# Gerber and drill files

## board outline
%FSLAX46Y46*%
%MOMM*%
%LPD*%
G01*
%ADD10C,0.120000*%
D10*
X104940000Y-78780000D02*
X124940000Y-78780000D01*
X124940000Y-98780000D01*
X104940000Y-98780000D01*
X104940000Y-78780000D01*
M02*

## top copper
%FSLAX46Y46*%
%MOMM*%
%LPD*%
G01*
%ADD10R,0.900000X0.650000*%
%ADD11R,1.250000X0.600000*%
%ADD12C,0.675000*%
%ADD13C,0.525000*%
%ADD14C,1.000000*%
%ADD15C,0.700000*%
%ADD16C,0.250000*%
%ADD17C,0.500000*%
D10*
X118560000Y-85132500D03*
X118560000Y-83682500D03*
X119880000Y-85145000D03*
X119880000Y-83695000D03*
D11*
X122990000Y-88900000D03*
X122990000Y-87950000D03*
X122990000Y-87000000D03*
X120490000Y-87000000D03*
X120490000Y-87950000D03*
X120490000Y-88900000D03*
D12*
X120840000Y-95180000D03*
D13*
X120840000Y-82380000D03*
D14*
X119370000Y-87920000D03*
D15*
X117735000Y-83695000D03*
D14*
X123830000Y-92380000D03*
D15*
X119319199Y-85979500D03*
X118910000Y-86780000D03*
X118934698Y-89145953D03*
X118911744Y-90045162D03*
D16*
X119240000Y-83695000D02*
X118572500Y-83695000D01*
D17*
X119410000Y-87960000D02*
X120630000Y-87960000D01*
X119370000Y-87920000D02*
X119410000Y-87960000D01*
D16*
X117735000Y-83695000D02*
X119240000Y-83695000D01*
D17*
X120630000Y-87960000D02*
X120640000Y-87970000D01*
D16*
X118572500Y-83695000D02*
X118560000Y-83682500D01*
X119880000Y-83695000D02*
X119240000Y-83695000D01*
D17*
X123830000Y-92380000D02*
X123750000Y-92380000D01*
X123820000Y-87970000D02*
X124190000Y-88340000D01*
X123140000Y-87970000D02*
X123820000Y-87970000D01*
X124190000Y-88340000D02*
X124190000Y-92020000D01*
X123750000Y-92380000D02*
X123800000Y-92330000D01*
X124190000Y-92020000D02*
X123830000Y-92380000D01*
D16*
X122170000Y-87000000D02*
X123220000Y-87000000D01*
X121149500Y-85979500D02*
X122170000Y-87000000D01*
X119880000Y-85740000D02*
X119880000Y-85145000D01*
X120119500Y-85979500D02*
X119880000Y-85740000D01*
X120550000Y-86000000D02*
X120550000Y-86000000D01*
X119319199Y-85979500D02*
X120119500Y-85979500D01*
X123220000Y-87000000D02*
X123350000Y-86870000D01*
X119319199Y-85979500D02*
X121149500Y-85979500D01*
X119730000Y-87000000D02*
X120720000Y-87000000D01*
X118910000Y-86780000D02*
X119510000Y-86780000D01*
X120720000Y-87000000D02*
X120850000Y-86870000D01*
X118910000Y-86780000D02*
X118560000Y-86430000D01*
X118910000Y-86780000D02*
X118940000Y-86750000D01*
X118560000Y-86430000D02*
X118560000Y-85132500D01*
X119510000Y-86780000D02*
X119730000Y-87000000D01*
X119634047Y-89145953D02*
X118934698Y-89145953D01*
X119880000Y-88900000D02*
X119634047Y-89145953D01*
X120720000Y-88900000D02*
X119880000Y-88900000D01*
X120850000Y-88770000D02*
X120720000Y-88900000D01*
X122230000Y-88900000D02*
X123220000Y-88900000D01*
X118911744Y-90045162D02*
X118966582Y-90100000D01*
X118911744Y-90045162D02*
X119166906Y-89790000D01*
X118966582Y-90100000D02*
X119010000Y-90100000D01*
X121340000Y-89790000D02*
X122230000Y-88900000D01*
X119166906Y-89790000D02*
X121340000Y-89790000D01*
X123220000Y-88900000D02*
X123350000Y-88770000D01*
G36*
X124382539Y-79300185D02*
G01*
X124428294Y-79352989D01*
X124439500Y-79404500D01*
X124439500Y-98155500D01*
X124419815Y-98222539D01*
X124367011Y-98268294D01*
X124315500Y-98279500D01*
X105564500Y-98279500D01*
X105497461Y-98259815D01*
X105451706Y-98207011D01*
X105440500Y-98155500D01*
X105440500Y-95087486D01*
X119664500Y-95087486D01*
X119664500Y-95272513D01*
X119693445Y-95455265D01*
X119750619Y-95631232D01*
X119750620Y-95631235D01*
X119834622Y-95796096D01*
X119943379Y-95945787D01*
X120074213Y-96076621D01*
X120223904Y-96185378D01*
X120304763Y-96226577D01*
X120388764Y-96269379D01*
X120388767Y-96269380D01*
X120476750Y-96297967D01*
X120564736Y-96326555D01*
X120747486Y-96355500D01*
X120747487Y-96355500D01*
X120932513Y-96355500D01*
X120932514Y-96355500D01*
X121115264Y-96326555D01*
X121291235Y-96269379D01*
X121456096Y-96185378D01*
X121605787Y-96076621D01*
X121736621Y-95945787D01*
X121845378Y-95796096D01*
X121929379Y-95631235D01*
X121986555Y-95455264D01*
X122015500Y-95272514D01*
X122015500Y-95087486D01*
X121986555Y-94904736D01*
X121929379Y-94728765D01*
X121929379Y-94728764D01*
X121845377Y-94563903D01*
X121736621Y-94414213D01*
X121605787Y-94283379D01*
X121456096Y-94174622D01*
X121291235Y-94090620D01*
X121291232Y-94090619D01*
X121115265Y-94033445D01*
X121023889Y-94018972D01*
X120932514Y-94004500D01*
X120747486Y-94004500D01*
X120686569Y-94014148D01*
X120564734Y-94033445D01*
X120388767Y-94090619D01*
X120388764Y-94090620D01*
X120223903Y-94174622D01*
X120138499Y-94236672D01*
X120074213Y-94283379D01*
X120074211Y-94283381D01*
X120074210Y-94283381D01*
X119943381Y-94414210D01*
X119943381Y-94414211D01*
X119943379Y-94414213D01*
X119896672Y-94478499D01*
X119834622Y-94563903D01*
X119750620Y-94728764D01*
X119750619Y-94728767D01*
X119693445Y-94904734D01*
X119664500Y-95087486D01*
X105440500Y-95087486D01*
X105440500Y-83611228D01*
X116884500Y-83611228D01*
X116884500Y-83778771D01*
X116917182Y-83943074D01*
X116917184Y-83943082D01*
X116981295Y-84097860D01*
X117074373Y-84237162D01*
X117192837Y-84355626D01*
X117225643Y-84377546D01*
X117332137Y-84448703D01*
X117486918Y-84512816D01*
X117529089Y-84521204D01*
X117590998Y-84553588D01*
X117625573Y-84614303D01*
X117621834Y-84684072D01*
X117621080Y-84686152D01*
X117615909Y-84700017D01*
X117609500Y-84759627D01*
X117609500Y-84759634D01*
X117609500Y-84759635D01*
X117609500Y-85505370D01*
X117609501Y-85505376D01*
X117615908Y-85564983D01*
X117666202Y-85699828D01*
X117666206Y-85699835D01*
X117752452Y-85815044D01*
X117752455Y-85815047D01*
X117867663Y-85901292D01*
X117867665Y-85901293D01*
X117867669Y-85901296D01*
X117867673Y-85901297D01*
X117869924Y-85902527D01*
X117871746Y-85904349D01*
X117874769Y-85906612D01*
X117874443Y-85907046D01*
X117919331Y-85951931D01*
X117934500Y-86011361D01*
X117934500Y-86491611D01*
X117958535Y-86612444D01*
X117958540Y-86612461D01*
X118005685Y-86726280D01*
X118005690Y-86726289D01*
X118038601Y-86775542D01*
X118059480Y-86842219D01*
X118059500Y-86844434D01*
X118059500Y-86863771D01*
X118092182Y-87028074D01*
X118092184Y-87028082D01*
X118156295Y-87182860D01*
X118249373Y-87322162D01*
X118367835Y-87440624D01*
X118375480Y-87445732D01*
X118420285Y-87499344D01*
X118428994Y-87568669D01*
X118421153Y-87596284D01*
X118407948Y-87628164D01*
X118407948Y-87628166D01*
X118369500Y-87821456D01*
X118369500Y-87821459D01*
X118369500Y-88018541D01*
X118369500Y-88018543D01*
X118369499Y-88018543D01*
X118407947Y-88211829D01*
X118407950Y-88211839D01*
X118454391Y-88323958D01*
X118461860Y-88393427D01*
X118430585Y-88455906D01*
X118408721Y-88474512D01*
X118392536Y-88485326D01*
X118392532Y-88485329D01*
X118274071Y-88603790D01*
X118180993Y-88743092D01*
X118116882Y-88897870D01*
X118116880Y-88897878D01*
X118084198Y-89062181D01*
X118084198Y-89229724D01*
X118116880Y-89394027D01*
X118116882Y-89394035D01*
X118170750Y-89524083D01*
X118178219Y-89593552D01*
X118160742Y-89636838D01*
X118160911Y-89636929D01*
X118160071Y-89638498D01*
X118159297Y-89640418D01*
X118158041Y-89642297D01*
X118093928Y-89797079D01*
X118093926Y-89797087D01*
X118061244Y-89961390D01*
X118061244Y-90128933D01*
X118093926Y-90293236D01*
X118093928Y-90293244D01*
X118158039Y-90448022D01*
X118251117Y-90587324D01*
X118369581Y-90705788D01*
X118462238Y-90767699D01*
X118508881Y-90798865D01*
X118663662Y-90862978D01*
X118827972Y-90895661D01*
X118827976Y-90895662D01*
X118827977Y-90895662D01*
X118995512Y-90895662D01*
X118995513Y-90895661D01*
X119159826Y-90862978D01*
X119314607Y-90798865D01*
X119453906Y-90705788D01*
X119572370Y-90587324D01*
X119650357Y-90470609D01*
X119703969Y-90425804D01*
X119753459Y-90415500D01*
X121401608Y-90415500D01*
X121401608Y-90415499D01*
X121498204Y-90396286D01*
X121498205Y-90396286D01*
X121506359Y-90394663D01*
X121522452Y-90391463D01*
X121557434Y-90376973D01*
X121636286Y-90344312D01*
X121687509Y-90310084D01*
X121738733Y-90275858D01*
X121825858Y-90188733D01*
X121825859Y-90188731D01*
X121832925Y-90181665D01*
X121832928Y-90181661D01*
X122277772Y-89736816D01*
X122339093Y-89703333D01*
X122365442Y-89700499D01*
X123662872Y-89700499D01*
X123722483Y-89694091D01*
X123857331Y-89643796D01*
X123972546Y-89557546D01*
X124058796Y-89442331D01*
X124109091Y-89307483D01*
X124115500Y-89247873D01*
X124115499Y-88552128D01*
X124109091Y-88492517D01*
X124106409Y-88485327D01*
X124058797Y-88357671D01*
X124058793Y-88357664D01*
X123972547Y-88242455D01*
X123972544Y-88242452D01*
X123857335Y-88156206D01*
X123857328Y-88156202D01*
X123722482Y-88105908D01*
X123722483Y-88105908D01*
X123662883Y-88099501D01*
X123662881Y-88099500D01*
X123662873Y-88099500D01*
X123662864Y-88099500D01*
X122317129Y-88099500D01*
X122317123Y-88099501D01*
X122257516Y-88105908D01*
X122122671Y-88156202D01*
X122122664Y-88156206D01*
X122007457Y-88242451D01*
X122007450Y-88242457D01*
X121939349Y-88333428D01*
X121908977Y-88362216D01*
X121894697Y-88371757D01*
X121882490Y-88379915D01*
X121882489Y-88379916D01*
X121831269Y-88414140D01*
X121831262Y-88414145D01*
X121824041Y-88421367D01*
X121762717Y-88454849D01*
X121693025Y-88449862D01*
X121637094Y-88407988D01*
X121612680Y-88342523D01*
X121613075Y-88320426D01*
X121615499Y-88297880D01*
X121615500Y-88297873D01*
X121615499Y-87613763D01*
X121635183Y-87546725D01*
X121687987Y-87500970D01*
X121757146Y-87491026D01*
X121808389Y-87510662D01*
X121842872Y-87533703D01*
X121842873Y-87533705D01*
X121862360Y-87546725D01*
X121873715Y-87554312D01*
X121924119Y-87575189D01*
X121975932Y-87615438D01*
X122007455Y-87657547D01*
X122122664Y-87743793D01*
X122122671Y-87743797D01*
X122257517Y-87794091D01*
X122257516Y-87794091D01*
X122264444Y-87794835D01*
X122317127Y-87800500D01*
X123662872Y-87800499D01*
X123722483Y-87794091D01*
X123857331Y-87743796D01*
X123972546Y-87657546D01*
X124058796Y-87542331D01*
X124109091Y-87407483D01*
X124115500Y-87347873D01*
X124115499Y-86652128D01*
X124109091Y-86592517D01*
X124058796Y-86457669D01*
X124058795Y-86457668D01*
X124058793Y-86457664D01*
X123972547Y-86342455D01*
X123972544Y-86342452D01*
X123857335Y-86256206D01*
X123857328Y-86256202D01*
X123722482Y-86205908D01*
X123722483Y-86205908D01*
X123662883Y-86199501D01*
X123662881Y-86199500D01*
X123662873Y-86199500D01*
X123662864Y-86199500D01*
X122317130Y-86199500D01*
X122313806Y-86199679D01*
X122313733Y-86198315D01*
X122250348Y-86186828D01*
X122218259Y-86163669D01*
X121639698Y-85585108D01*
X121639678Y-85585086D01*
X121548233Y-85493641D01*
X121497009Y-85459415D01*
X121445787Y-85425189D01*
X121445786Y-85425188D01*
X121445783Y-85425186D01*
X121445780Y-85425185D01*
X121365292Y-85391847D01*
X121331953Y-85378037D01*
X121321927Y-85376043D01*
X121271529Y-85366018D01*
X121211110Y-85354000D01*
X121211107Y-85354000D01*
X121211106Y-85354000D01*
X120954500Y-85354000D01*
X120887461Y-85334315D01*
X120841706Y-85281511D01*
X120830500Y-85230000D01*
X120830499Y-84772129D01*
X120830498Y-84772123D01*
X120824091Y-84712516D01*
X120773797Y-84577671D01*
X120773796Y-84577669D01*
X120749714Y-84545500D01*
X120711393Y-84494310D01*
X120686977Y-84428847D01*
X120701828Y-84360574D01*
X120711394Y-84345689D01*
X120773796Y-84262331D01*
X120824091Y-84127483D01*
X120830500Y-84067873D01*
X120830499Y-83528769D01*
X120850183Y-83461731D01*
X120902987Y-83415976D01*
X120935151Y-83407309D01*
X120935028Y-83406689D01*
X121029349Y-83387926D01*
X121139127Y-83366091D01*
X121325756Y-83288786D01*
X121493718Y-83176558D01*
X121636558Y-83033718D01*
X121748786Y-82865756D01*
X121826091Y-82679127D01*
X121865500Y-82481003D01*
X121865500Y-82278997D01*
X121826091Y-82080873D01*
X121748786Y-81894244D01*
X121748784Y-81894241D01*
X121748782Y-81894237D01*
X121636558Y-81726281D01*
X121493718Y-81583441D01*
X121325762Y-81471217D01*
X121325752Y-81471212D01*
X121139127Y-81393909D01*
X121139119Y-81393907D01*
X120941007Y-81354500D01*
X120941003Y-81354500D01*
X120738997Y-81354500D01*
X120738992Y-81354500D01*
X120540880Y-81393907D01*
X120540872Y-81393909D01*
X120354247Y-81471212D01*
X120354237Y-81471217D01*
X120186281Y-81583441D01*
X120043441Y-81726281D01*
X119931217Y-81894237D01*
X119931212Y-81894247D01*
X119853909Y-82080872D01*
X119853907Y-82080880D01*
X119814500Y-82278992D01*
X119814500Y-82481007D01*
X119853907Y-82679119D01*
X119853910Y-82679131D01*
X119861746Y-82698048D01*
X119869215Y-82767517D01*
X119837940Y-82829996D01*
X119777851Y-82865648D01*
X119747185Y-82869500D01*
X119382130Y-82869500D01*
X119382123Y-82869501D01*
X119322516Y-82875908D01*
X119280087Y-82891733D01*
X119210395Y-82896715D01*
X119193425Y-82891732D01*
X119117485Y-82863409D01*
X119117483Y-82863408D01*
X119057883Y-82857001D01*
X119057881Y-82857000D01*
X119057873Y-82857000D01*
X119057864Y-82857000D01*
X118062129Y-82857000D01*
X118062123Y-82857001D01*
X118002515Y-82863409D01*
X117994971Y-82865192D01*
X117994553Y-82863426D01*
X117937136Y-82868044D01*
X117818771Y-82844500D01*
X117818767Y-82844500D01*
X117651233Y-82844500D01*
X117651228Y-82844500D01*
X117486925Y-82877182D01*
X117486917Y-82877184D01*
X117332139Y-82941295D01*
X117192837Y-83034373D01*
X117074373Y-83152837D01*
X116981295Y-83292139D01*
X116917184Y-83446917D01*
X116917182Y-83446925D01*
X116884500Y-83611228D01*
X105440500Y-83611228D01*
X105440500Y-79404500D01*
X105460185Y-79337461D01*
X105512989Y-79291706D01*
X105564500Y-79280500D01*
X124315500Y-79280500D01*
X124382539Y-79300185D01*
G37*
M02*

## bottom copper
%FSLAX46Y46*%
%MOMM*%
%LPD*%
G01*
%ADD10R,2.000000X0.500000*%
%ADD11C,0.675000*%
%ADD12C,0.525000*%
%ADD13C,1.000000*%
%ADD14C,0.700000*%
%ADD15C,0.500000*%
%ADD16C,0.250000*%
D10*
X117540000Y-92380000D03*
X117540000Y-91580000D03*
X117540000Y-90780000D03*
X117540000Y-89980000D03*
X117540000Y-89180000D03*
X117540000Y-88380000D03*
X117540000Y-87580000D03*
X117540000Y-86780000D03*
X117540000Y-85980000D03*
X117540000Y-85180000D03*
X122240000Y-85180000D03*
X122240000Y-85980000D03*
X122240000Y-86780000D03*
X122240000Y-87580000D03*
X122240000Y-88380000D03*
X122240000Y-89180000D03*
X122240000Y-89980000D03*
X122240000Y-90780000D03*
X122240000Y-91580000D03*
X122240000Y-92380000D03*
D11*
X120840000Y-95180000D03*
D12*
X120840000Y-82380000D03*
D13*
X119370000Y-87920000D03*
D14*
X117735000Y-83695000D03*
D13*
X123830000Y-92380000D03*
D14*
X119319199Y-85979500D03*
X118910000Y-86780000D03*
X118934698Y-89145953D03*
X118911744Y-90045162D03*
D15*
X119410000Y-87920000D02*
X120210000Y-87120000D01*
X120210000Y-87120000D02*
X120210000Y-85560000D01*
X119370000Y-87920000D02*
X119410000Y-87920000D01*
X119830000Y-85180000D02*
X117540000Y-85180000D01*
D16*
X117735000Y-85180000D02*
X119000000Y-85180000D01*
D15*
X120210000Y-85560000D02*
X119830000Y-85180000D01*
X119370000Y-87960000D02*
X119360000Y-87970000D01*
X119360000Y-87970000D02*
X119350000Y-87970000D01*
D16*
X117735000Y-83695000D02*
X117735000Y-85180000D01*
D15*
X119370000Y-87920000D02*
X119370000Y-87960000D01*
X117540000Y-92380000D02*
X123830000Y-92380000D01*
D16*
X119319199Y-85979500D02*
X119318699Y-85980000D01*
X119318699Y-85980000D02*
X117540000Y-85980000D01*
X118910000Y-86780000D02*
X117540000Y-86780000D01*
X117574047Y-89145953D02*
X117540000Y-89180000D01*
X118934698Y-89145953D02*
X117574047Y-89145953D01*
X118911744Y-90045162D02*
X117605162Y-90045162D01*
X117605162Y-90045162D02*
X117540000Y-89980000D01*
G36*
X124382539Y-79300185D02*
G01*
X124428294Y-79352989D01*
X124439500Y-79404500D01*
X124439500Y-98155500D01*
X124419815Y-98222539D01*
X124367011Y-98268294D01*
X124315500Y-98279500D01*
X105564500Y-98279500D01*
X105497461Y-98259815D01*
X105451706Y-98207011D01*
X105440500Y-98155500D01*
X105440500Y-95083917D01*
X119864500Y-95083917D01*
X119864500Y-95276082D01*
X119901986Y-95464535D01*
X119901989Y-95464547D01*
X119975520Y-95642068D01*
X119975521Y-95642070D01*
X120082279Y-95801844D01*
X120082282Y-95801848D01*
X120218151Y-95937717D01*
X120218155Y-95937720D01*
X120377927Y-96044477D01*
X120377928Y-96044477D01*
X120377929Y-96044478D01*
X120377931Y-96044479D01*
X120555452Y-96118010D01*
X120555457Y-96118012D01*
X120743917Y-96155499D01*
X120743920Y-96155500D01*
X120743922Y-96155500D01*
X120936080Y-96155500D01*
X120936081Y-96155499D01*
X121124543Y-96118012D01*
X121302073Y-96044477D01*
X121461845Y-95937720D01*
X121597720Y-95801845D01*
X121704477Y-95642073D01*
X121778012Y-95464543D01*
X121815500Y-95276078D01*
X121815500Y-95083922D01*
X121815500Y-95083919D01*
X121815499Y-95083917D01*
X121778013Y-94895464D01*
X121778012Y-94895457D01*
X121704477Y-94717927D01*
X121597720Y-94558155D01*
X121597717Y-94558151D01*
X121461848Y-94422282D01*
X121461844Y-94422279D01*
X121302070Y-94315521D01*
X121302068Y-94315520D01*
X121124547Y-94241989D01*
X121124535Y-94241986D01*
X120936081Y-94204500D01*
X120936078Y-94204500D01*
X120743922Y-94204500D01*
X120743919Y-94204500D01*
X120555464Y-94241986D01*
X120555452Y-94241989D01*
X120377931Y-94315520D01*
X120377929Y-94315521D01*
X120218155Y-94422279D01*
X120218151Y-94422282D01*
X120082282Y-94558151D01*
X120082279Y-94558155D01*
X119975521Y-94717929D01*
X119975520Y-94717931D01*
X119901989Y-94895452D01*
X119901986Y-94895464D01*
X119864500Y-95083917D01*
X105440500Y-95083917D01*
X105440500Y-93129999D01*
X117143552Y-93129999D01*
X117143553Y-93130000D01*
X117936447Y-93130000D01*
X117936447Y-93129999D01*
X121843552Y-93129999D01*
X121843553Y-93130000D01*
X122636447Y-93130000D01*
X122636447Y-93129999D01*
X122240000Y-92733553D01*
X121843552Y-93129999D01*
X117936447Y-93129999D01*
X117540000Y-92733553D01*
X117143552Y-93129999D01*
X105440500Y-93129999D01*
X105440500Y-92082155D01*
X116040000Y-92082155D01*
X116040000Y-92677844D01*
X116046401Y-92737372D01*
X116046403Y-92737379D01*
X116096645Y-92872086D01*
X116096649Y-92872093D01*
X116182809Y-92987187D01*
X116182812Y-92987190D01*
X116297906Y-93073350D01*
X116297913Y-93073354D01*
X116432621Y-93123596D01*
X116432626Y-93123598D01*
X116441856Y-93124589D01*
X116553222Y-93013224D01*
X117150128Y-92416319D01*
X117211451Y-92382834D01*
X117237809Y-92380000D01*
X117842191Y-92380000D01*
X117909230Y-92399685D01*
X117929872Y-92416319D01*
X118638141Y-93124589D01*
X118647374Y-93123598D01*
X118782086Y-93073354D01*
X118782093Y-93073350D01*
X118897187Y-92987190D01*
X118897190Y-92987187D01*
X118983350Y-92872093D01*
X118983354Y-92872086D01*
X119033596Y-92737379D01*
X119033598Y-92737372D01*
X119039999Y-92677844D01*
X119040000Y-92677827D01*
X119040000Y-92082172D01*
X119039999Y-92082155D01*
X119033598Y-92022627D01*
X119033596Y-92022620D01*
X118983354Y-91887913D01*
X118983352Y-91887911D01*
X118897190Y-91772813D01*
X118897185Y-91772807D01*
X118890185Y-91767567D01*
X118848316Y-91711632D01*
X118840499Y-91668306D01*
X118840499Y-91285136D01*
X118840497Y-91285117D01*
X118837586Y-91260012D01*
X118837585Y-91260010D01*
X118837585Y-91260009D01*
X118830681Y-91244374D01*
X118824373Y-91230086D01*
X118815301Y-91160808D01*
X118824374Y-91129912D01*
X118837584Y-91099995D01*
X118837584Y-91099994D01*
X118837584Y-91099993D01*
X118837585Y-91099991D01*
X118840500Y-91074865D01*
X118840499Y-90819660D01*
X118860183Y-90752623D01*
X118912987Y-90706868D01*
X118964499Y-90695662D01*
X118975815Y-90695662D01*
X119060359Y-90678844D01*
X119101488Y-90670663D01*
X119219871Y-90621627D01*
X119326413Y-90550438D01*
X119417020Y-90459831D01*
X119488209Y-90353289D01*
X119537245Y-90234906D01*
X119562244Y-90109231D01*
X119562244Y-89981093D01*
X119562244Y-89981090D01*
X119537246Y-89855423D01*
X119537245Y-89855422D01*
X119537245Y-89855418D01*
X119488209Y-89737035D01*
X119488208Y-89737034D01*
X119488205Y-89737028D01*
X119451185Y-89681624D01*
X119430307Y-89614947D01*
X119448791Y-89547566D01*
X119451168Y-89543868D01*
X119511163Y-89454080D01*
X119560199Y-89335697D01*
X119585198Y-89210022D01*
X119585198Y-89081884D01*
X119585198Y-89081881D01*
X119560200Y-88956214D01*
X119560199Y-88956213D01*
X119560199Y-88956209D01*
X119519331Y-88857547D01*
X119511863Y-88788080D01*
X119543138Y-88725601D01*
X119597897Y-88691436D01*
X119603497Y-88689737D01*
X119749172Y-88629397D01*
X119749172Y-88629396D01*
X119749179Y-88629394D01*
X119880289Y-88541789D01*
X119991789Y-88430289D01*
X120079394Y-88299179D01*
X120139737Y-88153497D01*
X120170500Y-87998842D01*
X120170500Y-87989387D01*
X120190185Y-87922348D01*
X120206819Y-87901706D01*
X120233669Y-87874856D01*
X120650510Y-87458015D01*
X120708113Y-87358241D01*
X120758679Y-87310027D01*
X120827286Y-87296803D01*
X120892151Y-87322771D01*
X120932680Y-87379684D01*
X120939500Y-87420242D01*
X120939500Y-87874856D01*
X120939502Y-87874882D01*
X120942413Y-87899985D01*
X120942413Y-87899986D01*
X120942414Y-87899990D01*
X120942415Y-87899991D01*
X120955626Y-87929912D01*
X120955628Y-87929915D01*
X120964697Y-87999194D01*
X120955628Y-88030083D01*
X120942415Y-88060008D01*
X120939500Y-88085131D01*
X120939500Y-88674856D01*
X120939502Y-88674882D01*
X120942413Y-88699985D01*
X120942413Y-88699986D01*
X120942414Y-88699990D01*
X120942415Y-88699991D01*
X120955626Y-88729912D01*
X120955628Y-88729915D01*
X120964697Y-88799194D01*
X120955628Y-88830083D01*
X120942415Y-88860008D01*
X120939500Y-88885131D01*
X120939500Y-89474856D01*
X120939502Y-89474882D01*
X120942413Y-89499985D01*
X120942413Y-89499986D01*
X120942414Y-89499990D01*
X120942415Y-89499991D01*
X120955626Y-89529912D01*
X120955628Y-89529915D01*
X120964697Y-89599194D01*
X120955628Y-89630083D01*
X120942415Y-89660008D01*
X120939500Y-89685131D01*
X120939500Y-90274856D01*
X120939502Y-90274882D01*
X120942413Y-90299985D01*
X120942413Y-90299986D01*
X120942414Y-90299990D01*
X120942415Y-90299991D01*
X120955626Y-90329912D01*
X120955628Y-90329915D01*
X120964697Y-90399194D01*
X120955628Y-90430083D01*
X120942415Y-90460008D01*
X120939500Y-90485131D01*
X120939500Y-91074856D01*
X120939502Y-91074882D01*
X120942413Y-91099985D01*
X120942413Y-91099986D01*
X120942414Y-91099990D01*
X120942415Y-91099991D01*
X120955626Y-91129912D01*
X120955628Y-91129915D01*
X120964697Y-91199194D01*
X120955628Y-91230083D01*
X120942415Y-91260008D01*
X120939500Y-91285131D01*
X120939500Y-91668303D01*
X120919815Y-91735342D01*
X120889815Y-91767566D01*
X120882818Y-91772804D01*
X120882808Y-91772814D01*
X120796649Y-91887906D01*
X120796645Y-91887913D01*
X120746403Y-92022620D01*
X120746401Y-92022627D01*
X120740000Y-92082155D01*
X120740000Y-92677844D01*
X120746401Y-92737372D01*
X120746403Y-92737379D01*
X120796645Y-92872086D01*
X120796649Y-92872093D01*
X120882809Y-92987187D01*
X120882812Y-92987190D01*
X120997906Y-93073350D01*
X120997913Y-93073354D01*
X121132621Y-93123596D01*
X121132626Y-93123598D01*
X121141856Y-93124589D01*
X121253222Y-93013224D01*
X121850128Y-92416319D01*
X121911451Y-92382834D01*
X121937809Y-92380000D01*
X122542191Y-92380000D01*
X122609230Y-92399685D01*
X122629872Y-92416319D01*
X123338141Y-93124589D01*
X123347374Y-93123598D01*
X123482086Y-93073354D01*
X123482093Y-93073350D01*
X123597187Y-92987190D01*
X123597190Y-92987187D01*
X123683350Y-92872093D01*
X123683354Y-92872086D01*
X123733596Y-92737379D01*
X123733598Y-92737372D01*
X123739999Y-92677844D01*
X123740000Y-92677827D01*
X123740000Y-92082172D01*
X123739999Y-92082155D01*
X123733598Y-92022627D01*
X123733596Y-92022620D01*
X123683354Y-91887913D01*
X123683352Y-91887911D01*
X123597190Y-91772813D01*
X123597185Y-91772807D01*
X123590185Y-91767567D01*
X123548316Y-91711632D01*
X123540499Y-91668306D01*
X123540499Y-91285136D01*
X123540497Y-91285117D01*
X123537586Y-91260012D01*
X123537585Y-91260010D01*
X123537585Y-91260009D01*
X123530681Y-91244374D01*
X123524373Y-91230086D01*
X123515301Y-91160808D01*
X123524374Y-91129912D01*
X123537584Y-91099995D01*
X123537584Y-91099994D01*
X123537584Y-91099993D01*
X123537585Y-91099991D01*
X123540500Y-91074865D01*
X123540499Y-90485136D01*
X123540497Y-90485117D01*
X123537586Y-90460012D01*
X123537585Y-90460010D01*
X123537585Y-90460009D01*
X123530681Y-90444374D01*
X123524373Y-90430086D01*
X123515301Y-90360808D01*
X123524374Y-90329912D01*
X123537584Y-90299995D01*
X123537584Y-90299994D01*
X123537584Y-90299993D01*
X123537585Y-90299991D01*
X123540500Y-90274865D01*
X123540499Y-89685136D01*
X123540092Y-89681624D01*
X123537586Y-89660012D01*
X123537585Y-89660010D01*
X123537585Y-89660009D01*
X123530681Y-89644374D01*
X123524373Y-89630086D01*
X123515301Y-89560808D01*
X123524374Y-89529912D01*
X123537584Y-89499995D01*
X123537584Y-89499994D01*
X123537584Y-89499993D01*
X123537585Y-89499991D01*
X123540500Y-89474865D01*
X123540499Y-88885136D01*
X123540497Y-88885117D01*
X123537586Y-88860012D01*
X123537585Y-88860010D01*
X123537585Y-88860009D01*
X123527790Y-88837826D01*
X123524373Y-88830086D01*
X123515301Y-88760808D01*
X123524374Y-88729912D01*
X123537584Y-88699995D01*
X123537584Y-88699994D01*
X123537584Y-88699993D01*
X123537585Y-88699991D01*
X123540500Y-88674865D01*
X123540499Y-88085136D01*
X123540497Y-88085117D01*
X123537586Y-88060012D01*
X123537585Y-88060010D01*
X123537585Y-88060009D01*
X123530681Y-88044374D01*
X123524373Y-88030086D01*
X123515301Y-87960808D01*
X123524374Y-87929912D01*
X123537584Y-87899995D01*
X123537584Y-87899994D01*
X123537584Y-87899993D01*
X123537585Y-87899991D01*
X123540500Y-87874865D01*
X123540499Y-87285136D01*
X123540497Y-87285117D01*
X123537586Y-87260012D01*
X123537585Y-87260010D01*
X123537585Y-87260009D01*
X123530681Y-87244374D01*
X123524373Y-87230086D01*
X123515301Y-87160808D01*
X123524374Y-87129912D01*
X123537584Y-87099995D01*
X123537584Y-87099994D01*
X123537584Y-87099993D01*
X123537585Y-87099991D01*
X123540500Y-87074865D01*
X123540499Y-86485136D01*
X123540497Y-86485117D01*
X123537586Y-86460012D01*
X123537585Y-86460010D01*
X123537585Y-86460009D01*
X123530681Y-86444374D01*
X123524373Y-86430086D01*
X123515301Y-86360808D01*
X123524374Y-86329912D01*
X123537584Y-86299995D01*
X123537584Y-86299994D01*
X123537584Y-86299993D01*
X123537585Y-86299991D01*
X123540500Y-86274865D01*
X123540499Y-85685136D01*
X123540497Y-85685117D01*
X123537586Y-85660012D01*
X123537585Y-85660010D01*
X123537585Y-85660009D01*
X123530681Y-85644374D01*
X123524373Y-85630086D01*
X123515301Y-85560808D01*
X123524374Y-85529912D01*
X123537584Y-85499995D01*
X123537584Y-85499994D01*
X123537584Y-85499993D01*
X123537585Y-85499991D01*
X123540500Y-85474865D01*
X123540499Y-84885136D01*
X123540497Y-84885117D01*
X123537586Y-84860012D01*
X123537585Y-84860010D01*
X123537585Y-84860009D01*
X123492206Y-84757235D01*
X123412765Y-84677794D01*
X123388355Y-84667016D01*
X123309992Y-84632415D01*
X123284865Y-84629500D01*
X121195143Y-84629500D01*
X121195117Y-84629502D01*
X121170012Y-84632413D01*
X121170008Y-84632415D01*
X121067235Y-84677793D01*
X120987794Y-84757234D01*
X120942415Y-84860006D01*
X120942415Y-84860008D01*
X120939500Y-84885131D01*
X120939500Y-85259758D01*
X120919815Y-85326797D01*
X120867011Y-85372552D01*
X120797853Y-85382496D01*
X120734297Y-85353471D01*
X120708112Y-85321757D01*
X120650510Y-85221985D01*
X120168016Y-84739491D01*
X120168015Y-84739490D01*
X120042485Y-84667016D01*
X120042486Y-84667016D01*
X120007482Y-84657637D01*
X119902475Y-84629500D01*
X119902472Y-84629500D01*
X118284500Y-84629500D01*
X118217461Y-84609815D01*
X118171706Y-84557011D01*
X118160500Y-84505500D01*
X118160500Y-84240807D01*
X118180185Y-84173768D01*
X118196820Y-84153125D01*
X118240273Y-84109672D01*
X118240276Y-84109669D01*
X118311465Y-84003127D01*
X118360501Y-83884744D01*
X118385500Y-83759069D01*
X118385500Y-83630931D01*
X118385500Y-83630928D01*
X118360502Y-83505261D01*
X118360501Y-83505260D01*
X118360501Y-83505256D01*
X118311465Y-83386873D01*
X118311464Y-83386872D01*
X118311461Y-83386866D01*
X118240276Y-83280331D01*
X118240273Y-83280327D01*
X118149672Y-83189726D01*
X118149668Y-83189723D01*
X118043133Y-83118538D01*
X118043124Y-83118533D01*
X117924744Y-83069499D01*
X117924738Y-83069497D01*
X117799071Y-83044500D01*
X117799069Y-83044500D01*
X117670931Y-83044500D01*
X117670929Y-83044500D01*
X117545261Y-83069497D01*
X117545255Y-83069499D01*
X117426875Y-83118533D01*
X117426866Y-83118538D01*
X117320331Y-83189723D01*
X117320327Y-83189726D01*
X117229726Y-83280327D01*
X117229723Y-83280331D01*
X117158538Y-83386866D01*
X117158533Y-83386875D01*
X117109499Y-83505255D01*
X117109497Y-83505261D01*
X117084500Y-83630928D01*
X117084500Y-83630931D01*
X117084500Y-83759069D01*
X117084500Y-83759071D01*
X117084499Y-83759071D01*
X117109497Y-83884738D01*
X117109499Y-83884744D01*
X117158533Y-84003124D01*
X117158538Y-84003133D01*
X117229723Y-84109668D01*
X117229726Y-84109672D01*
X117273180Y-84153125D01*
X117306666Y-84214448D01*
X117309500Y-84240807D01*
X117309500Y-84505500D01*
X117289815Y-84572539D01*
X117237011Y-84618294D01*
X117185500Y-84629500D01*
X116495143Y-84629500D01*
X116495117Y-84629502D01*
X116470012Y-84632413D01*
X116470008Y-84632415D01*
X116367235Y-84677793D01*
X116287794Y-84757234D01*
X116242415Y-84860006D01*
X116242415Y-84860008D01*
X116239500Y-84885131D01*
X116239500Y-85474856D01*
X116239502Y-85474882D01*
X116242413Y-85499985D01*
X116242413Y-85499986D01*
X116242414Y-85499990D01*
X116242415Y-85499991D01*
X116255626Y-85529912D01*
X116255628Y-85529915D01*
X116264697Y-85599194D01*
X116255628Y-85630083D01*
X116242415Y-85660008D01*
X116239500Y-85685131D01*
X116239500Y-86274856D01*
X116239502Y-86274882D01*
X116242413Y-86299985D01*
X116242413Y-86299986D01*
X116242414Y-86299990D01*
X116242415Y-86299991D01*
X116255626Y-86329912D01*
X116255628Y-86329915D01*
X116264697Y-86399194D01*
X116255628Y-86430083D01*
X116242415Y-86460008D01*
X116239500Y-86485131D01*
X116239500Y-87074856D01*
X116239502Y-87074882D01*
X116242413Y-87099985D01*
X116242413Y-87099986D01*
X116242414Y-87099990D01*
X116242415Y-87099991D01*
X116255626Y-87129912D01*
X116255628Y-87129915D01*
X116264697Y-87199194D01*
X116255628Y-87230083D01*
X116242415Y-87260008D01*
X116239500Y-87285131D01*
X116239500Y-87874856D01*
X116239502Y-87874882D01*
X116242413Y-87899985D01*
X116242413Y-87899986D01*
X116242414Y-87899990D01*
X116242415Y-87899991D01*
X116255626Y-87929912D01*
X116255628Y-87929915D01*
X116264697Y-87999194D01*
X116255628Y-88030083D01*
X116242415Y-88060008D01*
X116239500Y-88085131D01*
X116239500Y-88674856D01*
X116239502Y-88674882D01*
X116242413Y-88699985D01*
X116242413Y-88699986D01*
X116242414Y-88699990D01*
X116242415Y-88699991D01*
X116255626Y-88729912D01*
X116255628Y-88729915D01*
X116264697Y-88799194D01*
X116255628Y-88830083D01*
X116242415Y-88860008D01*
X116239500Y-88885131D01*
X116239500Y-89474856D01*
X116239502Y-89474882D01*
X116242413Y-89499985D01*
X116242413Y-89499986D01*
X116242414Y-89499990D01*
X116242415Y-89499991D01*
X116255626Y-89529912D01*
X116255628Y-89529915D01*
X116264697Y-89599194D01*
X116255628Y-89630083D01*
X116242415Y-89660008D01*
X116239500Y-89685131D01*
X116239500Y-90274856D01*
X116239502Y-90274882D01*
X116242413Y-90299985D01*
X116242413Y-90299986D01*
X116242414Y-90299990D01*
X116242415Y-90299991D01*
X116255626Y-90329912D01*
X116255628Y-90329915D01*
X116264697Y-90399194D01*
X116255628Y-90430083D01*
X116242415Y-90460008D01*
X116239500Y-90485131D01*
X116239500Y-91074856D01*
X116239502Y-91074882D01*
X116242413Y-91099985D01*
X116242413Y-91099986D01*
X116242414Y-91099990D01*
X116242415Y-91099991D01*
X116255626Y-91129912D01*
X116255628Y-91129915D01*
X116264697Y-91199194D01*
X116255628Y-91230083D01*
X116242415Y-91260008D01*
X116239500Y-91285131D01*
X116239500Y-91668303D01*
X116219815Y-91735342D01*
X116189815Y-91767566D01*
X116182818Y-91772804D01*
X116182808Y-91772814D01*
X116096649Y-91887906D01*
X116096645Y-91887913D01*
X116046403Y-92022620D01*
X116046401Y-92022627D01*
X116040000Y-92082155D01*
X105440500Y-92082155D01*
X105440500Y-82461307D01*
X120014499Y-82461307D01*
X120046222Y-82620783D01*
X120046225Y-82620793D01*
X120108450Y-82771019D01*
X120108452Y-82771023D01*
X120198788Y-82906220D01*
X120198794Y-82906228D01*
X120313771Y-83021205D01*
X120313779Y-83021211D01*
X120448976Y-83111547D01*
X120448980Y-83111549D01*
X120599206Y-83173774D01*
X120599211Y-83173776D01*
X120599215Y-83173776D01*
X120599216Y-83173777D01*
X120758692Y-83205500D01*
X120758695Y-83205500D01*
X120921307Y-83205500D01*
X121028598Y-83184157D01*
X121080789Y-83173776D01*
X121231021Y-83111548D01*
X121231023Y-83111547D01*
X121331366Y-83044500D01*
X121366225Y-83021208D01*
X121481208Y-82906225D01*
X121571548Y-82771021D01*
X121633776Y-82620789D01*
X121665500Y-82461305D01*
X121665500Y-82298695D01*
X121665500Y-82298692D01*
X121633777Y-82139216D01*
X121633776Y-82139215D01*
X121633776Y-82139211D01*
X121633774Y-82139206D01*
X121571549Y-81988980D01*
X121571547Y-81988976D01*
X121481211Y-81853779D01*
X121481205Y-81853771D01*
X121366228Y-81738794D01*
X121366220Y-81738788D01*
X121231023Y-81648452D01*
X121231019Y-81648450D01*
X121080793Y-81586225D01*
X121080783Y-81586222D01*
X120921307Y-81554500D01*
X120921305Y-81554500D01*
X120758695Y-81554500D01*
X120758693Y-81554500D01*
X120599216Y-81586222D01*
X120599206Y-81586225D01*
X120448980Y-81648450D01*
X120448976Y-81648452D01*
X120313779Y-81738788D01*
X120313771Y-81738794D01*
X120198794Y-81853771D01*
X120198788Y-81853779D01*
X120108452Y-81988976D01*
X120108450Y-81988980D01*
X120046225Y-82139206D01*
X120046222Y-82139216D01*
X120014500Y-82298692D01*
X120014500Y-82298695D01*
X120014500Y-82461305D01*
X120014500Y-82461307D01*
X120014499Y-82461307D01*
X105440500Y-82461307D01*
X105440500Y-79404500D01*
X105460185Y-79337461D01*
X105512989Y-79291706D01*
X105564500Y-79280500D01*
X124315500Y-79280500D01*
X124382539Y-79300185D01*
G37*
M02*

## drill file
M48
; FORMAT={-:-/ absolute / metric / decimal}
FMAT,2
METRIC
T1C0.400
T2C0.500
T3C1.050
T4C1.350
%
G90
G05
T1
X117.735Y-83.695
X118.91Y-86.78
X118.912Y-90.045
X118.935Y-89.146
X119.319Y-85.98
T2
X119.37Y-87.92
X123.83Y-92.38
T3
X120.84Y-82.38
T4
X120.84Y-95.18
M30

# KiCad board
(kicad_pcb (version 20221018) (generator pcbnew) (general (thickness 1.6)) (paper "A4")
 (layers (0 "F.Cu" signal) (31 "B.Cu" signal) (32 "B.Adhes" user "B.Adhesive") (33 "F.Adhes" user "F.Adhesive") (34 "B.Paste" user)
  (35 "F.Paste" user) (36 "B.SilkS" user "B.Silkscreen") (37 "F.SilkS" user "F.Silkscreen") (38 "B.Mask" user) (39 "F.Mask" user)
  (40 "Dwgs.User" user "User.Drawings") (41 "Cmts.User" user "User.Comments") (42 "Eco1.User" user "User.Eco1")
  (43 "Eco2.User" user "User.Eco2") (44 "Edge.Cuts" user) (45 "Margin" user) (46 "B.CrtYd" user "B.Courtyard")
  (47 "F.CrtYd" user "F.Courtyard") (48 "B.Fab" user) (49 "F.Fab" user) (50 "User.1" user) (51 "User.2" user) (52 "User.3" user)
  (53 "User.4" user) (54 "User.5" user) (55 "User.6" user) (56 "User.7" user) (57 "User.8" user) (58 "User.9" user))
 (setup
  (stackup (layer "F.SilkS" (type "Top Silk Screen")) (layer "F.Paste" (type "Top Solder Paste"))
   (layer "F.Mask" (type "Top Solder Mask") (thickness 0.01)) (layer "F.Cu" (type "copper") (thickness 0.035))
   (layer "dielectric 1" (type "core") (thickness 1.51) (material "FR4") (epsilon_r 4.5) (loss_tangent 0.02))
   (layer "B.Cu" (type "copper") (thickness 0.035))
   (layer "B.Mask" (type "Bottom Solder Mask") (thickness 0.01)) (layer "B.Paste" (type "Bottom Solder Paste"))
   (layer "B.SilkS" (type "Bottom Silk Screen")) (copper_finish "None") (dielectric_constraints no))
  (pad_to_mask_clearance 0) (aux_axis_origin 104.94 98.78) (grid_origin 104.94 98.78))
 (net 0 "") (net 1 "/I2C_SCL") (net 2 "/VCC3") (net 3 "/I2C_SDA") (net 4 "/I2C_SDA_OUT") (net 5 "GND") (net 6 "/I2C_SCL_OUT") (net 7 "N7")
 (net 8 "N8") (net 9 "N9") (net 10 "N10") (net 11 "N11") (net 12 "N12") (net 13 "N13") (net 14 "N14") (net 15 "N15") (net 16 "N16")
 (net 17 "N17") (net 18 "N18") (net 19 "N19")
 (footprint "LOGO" (layer "F.Cu") (at 107.76 84.07)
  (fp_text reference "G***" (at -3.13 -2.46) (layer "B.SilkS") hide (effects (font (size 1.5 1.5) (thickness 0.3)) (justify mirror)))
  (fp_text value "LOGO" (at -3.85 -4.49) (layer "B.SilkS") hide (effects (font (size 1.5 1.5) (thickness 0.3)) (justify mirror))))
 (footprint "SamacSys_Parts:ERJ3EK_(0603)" (layer "F.Cu") (at 118.56 84.4075 90)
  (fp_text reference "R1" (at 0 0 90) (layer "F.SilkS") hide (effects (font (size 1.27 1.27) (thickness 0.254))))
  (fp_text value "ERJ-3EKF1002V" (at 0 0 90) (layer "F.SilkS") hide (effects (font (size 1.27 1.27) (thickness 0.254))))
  (pad "1" smd rect (at -0.725 0 90) (size 0.65 0.9) (layers "F.Cu" "F.Paste" "F.Mask") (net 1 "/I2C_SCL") (thermal_bridge_angle 45))
  (pad "2" smd rect (at 0.725 0 90) (size 0.65 0.9) (layers "F.Cu" "F.Paste" "F.Mask") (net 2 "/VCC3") (thermal_bridge_angle 45)))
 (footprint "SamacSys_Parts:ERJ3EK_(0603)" (layer "F.Cu") (at 119.88 84.42 90)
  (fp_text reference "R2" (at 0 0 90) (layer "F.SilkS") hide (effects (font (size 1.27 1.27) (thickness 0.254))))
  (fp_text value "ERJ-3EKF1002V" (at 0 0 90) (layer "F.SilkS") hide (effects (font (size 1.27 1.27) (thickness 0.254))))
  (pad "1" smd rect (at -0.725 0 90) (size 0.65 0.9) (layers "F.Cu" "F.Paste" "F.Mask") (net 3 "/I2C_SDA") (thermal_bridge_angle 45))
  (pad "2" smd rect (at 0.725 0 90) (size 0.65 0.9) (layers "F.Cu" "F.Paste" "F.Mask") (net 2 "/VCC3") (thermal_bridge_angle 45)))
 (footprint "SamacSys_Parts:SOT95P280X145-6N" (layer "F.Cu") (at 121.74 87.95 180)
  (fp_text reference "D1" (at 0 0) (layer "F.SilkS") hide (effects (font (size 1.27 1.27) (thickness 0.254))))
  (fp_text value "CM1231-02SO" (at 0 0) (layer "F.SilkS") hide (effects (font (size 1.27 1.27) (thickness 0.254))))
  (pad "1" smd rect (at -1.25 -0.95 270) (size 0.6 1.25) (layers "F.Cu" "F.Paste" "F.Mask") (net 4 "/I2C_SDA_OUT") (thermal_bridge_angle 45))
  (pad "2" smd rect (at -1.25 0 270) (size 0.6 1.25) (layers "F.Cu" "F.Paste" "F.Mask") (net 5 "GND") (thermal_bridge_angle 45))
  (pad "3" smd rect (at -1.25 0.95 270) (size 0.6 1.25) (layers "F.Cu" "F.Paste" "F.Mask") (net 3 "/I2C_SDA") (thermal_bridge_angle 45))
  (pad "4" smd rect (at 1.25 0.95 270) (size 0.6 1.25) (layers "F.Cu" "F.Paste" "F.Mask") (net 1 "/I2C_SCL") (thermal_bridge_angle 45))
  (pad "5" smd rect (at 1.25 0 270) (size 0.6 1.25) (layers "F.Cu" "F.Paste" "F.Mask") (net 2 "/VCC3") (thermal_bridge_angle 45))
  (pad "6" smd rect (at 1.25 -0.95 270) (size 0.6 1.25) (layers "F.Cu" "F.Paste" "F.Mask") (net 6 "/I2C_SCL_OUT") (thermal_bridge_angle 45)))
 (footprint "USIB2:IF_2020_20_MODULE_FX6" (layer "B.Cu") (at 114.94 88.78 -90)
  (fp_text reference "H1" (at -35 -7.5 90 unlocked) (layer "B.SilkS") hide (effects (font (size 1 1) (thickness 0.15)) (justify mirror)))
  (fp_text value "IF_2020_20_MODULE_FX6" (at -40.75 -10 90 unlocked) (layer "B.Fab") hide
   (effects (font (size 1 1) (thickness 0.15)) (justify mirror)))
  (fp_rect (start -10 10) (end 10 -10) (stroke (width 0.12) (type solid)) (fill none) (layer "Edge.Cuts"))
  (pad "1" smd rect (at 3.6 -2.6 270) (size 0.5 2) (layers "B.Cu" "B.Paste" "B.Mask") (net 5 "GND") (thermal_bridge_angle 45))
  (pad "2" smd rect (at 2.8 -2.6 270) (size 0.5 2) (layers "B.Cu" "B.Paste" "B.Mask") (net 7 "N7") (thermal_bridge_angle 45))
  (pad "3" smd rect (at 2 -2.6 270) (size 0.5 2) (layers "B.Cu" "B.Paste" "B.Mask") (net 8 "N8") (thermal_bridge_angle 45))
  (pad "4" smd rect (at 1.2 -2.6 270) (size 0.5 2) (layers "B.Cu" "B.Paste" "B.Mask") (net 4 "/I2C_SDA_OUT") (thermal_bridge_angle 45))
  (pad "5" smd rect (at 0.4 -2.6 270) (size 0.5 2) (layers "B.Cu" "B.Paste" "B.Mask") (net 6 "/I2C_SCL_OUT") (thermal_bridge_angle 45))
  (pad "6" smd rect (at -0.4 -2.6 270) (size 0.5 2) (layers "B.Cu" "B.Paste" "B.Mask") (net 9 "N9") (thermal_bridge_angle 45))
  (pad "7" smd rect (at -1.2 -2.6 270) (size 0.5 2) (layers "B.Cu" "B.Paste" "B.Mask") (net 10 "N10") (thermal_bridge_angle 45))
  (pad "8" smd rect (at -2 -2.6 270) (size 0.5 2) (layers "B.Cu" "B.Paste" "B.Mask") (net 1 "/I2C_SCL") (thermal_bridge_angle 45))
  (pad "9" smd rect (at -2.8 -2.6 270) (size 0.5 2) (layers "B.Cu" "B.Paste" "B.Mask") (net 3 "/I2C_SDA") (thermal_bridge_angle 45))
  (pad "10" smd rect (at -3.6 -2.6 270) (size 0.5 2) (layers "B.Cu" "B.Paste" "B.Mask") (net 2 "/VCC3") (thermal_bridge_angle 45))
  (pad "11" smd rect (at -3.6 -7.3 270) (size 0.5 2) (layers "B.Cu" "B.Paste" "B.Mask") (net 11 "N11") (thermal_bridge_angle 45))
  (pad "12" smd rect (at -2.8 -7.3 270) (size 0.5 2) (layers "B.Cu" "B.Paste" "B.Mask") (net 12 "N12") (thermal_bridge_angle 45))
  (pad "13" smd rect (at -2 -7.3 270) (size 0.5 2) (layers "B.Cu" "B.Paste" "B.Mask") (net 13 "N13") (thermal_bridge_angle 45))
  (pad "14" smd rect (at -1.2 -7.3 270) (size 0.5 2) (layers "B.Cu" "B.Paste" "B.Mask") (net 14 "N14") (thermal_bridge_angle 45))
  (pad "15" smd rect (at -0.4 -7.3 270) (size 0.5 2) (layers "B.Cu" "B.Paste" "B.Mask") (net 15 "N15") (thermal_bridge_angle 45))
  (pad "16" smd rect (at 0.4 -7.3 270) (size 0.5 2) (layers "B.Cu" "B.Paste" "B.Mask") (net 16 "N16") (thermal_bridge_angle 45))
  (pad "17" smd rect (at 1.2 -7.3 270) (size 0.5 2) (layers "B.Cu" "B.Paste" "B.Mask") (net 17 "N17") (thermal_bridge_angle 45))
  (pad "18" smd rect (at 2 -7.3 270) (size 0.5 2) (layers "B.Cu" "B.Paste" "B.Mask") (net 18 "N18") (thermal_bridge_angle 45))
  (pad "19" smd rect (at 2.8 -7.3 270) (size 0.5 2) (layers "B.Cu" "B.Paste" "B.Mask") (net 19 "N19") (thermal_bridge_angle 45))
  (pad "20" smd rect (at 3.6 -7.3 270) (size 0.5 2) (layers "B.Cu" "B.Paste" "B.Mask") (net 5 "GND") (thermal_bridge_angle 45))
  (pad "MH1" thru_hole circle (at 6.4 -5.9 180) (size 0.675 0.675) (drill 1.35) (layers "*.Cu" "*.Mask" "B.SilkS"))
  (pad "MH2" thru_hole circle (at -6.4 -5.9 180) (size 0.525 0.525) (drill 1.05) (layers "*.Cu" "*.Mask" "B.SilkS")))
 (segment (start 119.24 83.695) (end 118.5725 83.695) (width 0.25) (layer "F.Cu") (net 2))
 (segment (start 119.41 87.96) (end 120.63 87.96) (width 0.5) (layer "F.Cu") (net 2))
 (segment (start 119.37 87.92) (end 119.41 87.96) (width 0.5) (layer "F.Cu") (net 2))
 (segment (start 117.735 83.695) (end 119.24 83.695) (width 0.25) (layer "F.Cu") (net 2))
 (segment (start 120.63 87.96) (end 120.64 87.97) (width 0.5) (layer "F.Cu") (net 2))
 (segment (start 118.5725 83.695) (end 118.56 83.6825) (width 0.25) (layer "F.Cu") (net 2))
 (segment (start 119.88 83.695) (end 119.24 83.695) (width 0.25) (layer "F.Cu") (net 2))
 (via (at 119.37 87.92) (size 1) (drill 0.5) (layers "F.Cu" "B.Cu") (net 2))
 (via (at 117.735 83.695) (size 0.7) (drill 0.4) (layers "F.Cu" "B.Cu") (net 2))
 (segment (start 119.41 87.92) (end 120.21 87.12) (width 0.5) (layer "B.Cu") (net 2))
 (segment (start 120.21 87.12) (end 120.21 85.56) (width 0.5) (layer "B.Cu") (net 2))
 (segment (start 119.37 87.92) (end 119.41 87.92) (width 0.5) (layer "B.Cu") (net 2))
 (segment (start 119.83 85.18) (end 117.54 85.18) (width 0.5) (layer "B.Cu") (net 2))
 (segment (start 117.735 85.18) (end 119 85.18) (width 0.25) (layer "B.Cu") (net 2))
 (segment (start 120.21 85.56) (end 119.83 85.18) (width 0.5) (layer "B.Cu") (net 2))
 (segment (start 119.37 87.96) (end 119.36 87.97) (width 0.5) (layer "B.Cu") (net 2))
 (segment (start 119.36 87.97) (end 119.35 87.97) (width 0.5) (layer "B.Cu") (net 2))
 (segment (start 117.735 83.695) (end 117.735 85.18) (width 0.25) (layer "B.Cu") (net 2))
 (segment (start 119.37 87.92) (end 119.37 87.96) (width 0.5) (layer "B.Cu") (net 2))
 (segment (start 123.83 92.38) (end 123.75 92.38) (width 0.5) (layer "F.Cu") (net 5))
 (segment (start 123.82 87.97) (end 124.19 88.34) (width 0.5) (layer "F.Cu") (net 5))
 (segment (start 123.14 87.97) (end 123.82 87.97) (width 0.5) (layer "F.Cu") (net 5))
 (segment (start 124.19 88.34) (end 124.19 92.02) (width 0.5) (layer "F.Cu") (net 5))
 (segment (start 123.75 92.38) (end 123.8 92.33) (width 0.5) (layer "F.Cu") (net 5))
 (segment (start 124.19 92.02) (end 123.83 92.38) (width 0.5) (layer "F.Cu") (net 5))
 (via (at 123.83 92.38) (size 1) (drill 0.5) (layers "F.Cu" "B.Cu") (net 5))
 (segment (start 117.54 92.38) (end 123.83 92.38) (width 0.5) (layer "B.Cu") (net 5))
 (segment (start 122.17 87) (end 123.22 87) (width 0.25) (layer "F.Cu") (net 3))
 (segment (start 121.1495 85.9795) (end 122.17 87) (width 0.25) (layer "F.Cu") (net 3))
 (segment (start 119.88 85.74) (end 119.88 85.145) (width 0.25) (layer "F.Cu") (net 3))
 (segment (start 120.1195 85.9795) (end 119.88 85.74) (width 0.25) (layer "F.Cu") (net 3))
 (segment (start 120.55 86) (end 120.55 86) (width 0.25) (layer "F.Cu") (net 3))
 (segment (start 119.319199 85.9795) (end 120.1195 85.9795) (width 0.25) (layer "F.Cu") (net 3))
 (segment (start 123.22 87) (end 123.35 86.87) (width 0.25) (layer "F.Cu") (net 3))
 (segment (start 119.319199 85.9795) (end 121.1495 85.9795) (width 0.25) (layer "F.Cu") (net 3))
 (via (at 119.319199 85.9795) (size 0.7) (drill 0.4) (layers "F.Cu" "B.Cu") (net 3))
 (segment (start 119.319199 85.9795) (end 119.318699 85.98) (width 0.25) (layer "B.Cu") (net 3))
 (segment (start 119.318699 85.98) (end 117.54 85.98) (width 0.25) (layer "B.Cu") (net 3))
 (segment (start 119.73 87) (end 120.72 87) (width 0.25) (layer "F.Cu") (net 1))
 (segment (start 118.91 86.78) (end 119.51 86.78) (width 0.25) (layer "F.Cu") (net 1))
 (segment (start 120.72 87) (end 120.85 86.87) (width 0.25) (layer "F.Cu") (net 1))
 (segment (start 118.91 86.78) (end 118.56 86.43) (width 0.25) (layer "F.Cu") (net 1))
 (segment (start 118.91 86.78) (end 118.94 86.75) (width 0.25) (layer "F.Cu") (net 1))
 (segment (start 118.56 86.43) (end 118.56 85.1325) (width 0.25) (layer "F.Cu") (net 1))
 (segment (start 119.51 86.78) (end 119.73 87) (width 0.25) (layer "F.Cu") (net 1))
 (via (at 118.91 86.78) (size 0.7) (drill 0.4) (layers "F.Cu" "B.Cu") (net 1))
 (segment (start 118.91 86.78) (end 117.54 86.78) (width 0.25) (layer "B.Cu") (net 1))
 (segment (start 119.634047 89.145953) (end 118.934698 89.145953) (width 0.25) (layer "F.Cu") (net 6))
 (segment (start 119.88 88.9) (end 119.634047 89.145953) (width 0.25) (layer "F.Cu") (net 6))
 (segment (start 120.72 88.9) (end 119.88 88.9) (width 0.25) (layer "F.Cu") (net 6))
 (segment (start 120.85 88.77) (end 120.72 88.9) (width 0.25) (layer "F.Cu") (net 6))
 (via (at 118.934698 89.145953) (size 0.7) (drill 0.4) (layers "F.Cu" "B.Cu") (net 6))
 (segment (start 117.574047 89.145953) (end 117.54 89.18) (width 0.25) (layer "B.Cu") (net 6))
 (segment (start 118.934698 89.145953) (end 117.574047 89.145953) (width 0.25) (layer "B.Cu") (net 6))
 (segment (start 122.23 88.9) (end 123.22 88.9) (width 0.25) (layer "F.Cu") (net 4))
 (segment (start 118.911744 90.045162) (end 118.966582 90.1) (width 0.25) (layer "F.Cu") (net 4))
 (segment (start 118.911744 90.045162) (end 119.166906 89.79) (width 0.25) (layer "F.Cu") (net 4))
 (segment (start 118.966582 90.1) (end 119.01 90.1) (width 0.25) (layer "F.Cu") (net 4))
 (segment (start 121.34 89.79) (end 122.23 88.9) (width 0.25) (layer "F.Cu") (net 4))
 (segment (start 119.166906 89.79) (end 121.34 89.79) (width 0.25) (layer "F.Cu") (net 4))
 (segment (start 123.22 88.9) (end 123.35 88.77) (width 0.25) (layer "F.Cu") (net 4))
 (via (at 118.911744 90.045162) (size 0.7) (drill 0.4) (layers "F.Cu" "B.Cu") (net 4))
 (segment (start 118.911744 90.045162) (end 117.605162 90.045162) (width 0.25) (layer "B.Cu") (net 4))
 (segment (start 117.605162 90.045162) (end 117.54 89.98) (width 0.25) (layer "B.Cu") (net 4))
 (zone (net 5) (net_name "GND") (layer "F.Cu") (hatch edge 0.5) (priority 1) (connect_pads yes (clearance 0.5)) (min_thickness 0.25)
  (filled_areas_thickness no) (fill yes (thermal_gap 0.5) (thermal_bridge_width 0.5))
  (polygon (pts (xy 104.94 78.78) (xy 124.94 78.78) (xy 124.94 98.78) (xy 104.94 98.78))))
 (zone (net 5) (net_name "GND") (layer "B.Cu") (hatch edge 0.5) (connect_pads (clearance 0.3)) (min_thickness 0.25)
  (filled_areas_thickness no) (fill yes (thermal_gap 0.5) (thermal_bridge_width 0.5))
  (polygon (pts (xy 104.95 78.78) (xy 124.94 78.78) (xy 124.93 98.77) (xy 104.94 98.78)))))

